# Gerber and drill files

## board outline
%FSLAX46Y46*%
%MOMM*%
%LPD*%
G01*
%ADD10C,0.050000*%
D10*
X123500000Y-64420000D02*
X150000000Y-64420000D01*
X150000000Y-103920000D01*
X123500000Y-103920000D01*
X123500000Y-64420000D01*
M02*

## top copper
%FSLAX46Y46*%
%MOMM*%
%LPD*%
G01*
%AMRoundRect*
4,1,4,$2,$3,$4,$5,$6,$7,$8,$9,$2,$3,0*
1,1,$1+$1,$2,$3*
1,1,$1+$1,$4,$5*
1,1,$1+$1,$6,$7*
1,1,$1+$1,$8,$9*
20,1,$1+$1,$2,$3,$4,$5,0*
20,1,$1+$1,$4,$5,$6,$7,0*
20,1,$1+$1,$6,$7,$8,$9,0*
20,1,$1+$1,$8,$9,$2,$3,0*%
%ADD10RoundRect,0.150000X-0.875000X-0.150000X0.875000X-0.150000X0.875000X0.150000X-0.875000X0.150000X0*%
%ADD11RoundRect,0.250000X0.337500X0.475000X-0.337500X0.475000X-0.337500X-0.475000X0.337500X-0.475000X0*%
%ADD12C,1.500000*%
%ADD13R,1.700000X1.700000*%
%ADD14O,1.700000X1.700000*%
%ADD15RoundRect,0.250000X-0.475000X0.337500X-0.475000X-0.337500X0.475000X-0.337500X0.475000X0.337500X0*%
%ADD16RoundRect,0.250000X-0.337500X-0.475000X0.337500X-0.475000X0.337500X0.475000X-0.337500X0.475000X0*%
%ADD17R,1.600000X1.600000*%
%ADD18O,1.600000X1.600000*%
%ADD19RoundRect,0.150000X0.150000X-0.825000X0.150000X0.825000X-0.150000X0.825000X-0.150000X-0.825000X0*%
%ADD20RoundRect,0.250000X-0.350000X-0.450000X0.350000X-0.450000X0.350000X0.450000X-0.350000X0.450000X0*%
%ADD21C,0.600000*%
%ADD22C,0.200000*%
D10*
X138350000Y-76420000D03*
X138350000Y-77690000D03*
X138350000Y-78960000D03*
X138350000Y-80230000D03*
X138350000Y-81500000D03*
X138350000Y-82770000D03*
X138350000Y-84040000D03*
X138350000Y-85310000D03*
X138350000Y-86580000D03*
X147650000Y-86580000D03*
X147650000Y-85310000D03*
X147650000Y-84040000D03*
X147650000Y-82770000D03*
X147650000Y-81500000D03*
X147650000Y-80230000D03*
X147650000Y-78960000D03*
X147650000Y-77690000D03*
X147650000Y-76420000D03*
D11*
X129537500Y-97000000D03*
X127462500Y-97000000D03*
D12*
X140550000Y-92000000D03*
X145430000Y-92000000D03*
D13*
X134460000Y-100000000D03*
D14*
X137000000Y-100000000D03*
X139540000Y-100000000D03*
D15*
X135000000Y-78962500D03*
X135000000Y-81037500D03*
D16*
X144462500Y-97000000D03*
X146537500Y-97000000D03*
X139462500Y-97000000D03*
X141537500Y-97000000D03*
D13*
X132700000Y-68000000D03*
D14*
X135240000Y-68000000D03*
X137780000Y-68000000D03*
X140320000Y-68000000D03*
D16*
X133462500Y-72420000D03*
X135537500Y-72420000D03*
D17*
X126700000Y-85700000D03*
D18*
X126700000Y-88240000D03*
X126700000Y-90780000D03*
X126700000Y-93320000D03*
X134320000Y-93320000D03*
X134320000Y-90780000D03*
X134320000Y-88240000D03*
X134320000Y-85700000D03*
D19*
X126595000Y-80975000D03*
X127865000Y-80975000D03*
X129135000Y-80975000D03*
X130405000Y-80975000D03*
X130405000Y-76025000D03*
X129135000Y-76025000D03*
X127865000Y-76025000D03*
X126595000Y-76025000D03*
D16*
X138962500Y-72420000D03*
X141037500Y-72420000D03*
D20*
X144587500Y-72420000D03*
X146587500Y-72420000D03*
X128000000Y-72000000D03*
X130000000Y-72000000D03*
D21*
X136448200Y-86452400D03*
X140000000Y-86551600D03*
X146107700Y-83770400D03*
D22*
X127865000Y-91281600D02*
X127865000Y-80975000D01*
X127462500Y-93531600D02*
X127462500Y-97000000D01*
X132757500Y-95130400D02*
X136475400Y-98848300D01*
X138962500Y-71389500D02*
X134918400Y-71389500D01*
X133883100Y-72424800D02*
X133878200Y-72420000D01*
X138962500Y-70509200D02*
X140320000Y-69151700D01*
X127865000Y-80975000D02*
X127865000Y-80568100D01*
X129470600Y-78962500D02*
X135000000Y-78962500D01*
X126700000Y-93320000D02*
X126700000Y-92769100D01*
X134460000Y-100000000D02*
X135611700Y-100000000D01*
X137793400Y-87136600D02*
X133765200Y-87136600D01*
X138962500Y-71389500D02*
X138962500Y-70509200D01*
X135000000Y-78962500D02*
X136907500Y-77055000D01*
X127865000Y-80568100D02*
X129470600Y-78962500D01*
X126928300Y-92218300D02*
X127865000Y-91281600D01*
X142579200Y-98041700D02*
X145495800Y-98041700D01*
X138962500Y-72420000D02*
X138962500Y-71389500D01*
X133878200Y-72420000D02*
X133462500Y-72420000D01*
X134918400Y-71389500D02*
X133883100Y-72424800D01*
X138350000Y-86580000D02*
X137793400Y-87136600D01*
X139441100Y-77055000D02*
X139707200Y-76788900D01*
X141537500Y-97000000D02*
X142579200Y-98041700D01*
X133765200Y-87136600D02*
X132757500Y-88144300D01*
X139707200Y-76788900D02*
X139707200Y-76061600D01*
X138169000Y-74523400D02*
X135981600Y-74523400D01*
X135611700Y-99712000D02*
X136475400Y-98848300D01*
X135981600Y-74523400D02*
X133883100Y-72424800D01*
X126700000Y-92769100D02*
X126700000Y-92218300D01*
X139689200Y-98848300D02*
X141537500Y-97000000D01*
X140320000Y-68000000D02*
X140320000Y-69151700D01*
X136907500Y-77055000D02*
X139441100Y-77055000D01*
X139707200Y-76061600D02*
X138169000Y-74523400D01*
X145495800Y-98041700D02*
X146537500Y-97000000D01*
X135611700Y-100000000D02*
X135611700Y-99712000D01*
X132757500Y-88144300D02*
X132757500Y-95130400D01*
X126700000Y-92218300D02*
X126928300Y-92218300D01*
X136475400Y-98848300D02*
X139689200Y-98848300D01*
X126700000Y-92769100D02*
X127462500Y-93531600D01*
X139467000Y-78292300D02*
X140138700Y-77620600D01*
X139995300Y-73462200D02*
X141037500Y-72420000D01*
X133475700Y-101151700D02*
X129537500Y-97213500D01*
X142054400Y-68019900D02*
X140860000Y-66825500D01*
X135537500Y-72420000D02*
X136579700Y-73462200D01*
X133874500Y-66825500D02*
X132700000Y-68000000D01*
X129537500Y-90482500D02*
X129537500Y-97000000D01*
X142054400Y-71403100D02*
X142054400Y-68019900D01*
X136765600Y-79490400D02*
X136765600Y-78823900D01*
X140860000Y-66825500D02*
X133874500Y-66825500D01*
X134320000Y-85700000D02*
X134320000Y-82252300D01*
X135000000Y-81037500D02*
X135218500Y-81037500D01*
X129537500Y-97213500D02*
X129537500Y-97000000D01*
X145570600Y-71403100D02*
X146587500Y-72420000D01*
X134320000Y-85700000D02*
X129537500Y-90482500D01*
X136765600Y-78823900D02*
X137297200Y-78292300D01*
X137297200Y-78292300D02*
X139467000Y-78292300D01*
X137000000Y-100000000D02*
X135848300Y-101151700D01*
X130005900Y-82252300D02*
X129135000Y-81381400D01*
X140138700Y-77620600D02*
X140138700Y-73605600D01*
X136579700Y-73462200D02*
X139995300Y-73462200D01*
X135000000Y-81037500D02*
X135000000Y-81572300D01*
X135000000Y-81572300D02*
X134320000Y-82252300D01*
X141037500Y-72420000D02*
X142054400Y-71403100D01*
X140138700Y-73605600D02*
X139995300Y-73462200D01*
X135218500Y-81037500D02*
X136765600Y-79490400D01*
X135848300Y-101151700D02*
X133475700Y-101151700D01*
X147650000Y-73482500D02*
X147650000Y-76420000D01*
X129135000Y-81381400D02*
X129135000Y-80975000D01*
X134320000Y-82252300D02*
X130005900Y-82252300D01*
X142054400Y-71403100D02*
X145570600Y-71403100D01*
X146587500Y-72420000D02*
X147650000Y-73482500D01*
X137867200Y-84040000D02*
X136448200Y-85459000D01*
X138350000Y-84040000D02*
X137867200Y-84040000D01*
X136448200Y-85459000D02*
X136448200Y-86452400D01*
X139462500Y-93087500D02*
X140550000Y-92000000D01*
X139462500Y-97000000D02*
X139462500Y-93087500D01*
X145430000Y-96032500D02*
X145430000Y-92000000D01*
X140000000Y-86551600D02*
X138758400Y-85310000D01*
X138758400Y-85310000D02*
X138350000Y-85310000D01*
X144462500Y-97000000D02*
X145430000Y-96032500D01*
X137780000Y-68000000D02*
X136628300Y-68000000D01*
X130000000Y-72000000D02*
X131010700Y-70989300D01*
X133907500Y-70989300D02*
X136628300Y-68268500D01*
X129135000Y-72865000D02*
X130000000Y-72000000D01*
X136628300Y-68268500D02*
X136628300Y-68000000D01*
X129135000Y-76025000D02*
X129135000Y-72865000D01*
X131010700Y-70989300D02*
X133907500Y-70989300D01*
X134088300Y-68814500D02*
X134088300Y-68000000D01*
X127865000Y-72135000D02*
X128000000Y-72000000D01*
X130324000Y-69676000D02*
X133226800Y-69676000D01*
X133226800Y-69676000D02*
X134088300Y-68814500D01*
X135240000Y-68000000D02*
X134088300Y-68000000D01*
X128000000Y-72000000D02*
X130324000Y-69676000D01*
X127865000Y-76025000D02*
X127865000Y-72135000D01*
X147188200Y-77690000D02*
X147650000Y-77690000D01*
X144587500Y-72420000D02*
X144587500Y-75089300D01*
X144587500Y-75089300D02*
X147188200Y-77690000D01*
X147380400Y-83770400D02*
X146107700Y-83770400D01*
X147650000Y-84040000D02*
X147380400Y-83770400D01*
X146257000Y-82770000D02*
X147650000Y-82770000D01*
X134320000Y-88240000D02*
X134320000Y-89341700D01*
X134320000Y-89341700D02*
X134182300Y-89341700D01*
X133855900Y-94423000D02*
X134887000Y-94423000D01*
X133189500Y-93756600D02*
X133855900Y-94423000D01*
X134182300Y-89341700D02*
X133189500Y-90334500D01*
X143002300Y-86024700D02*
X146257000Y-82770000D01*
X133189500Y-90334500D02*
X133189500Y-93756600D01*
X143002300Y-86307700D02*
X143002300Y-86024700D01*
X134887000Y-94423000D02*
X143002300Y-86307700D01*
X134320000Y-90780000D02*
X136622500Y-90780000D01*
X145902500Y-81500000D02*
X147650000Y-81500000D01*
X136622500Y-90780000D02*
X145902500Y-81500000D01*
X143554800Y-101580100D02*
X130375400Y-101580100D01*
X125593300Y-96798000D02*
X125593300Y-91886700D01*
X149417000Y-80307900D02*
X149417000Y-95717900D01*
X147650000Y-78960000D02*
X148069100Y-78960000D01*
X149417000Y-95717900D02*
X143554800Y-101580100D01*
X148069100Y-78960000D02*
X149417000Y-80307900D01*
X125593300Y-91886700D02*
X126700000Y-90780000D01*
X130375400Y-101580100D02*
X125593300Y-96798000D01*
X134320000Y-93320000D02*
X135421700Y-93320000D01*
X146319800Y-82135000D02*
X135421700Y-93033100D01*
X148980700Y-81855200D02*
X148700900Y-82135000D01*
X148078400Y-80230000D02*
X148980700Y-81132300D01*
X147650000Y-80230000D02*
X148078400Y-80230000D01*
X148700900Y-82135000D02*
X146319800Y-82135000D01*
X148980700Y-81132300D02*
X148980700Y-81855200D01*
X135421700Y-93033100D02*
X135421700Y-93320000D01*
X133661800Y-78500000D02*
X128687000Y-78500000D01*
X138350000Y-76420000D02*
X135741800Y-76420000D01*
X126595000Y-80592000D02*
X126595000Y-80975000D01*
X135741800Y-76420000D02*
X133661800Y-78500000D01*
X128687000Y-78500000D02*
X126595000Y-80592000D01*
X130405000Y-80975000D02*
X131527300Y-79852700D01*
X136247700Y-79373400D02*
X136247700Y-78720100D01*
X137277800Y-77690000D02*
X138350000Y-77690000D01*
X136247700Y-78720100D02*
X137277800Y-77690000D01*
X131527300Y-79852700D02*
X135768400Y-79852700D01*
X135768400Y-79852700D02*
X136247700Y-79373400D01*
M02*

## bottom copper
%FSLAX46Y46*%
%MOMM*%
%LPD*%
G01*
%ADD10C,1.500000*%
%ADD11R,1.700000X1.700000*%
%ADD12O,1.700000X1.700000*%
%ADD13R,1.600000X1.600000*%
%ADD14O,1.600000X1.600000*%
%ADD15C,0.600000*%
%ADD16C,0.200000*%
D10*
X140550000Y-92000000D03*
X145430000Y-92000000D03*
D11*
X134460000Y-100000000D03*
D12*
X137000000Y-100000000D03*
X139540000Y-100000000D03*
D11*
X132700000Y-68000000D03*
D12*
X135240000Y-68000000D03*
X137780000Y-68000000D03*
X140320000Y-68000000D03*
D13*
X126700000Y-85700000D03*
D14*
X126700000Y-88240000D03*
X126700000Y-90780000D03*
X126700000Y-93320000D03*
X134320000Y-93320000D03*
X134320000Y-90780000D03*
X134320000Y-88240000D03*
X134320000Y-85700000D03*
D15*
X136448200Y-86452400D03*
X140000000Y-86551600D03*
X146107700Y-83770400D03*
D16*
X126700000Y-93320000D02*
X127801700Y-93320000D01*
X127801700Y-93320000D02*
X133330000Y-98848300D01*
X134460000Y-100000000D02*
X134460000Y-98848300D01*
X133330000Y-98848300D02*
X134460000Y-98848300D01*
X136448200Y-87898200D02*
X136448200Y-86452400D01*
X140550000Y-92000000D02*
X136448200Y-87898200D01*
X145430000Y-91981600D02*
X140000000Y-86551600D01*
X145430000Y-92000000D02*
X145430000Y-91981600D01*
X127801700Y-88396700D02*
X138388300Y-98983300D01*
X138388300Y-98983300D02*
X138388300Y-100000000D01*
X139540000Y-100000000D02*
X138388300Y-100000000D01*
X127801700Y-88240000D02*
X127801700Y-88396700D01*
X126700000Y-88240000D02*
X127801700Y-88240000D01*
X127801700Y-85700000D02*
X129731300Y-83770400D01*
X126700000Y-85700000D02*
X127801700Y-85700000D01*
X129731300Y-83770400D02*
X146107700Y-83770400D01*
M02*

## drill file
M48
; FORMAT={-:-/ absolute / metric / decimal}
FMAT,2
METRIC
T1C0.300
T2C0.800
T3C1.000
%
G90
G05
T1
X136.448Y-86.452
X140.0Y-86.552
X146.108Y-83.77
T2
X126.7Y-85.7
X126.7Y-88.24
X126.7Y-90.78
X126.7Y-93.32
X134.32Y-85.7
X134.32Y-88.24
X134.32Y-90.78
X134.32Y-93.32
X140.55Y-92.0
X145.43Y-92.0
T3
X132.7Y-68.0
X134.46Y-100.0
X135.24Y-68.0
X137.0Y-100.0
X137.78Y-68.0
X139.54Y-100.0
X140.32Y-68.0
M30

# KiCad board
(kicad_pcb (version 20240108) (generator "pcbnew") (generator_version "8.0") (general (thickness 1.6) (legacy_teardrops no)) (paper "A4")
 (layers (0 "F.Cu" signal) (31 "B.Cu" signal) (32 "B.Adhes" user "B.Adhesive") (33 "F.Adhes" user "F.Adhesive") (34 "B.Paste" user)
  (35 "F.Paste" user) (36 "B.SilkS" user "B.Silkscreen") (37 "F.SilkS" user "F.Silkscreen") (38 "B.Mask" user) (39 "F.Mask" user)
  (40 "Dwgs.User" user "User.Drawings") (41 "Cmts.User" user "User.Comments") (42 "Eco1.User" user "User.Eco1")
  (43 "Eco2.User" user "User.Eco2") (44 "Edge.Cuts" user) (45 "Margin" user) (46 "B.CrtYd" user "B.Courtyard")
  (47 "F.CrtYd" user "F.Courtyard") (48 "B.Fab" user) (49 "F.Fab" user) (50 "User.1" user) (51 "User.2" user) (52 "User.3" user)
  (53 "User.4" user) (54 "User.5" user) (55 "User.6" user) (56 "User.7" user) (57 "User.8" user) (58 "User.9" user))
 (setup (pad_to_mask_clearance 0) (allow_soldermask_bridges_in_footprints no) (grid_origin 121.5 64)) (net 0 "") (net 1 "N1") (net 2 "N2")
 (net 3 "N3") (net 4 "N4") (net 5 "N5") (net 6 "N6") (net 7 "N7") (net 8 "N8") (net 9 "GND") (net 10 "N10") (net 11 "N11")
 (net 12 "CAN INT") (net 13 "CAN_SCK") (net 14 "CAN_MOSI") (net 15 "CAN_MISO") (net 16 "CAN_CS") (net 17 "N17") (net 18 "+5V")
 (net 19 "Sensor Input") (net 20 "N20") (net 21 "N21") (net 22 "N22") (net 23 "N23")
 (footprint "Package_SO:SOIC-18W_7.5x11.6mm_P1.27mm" (layer "F.Cu") (at 143 81.5)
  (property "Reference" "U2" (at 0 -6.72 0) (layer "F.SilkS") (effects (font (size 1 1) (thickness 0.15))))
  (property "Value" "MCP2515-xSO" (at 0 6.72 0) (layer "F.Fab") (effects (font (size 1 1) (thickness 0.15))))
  (pad "1" smd roundrect (at -4.65 -5.08) (size 2.05 0.6) (layers "F.Cu" "F.Paste" "F.Mask") (roundrect_rratio 0.25) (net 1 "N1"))
  (pad "2" smd roundrect (at -4.65 -3.81) (size 2.05 0.6) (layers "F.Cu" "F.Paste" "F.Mask") (roundrect_rratio 0.25) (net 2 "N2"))
  (pad "3" smd roundrect (at -4.65 -2.54) (size 2.05 0.6) (layers "F.Cu" "F.Paste" "F.Mask") (roundrect_rratio 0.25) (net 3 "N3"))
  (pad "4" smd roundrect (at -4.65 -1.27) (size 2.05 0.6) (layers "F.Cu" "F.Paste" "F.Mask") (roundrect_rratio 0.25) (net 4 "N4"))
  (pad "5" smd roundrect (at -4.65 0) (size 2.05 0.6) (layers "F.Cu" "F.Paste" "F.Mask") (roundrect_rratio 0.25) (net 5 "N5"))
  (pad "6" smd roundrect (at -4.65 1.27) (size 2.05 0.6) (layers "F.Cu" "F.Paste" "F.Mask") (roundrect_rratio 0.25) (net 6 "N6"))
  (pad "7" smd roundrect (at -4.65 2.54) (size 2.05 0.6) (layers "F.Cu" "F.Paste" "F.Mask") (roundrect_rratio 0.25) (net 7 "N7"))
  (pad "8" smd roundrect (at -4.65 3.81) (size 2.05 0.6) (layers "F.Cu" "F.Paste" "F.Mask") (roundrect_rratio 0.25) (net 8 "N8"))
  (pad "9" smd roundrect (at -4.65 5.08) (size 2.05 0.6) (layers "F.Cu" "F.Paste" "F.Mask") (roundrect_rratio 0.25) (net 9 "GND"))
  (pad "10" smd roundrect (at 4.65 5.08) (size 2.05 0.6) (layers "F.Cu" "F.Paste" "F.Mask") (roundrect_rratio 0.25) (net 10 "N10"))
  (pad "11" smd roundrect (at 4.65 3.81) (size 2.05 0.6) (layers "F.Cu" "F.Paste" "F.Mask") (roundrect_rratio 0.25) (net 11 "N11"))
  (pad "12" smd roundrect (at 4.65 2.54) (size 2.05 0.6) (layers "F.Cu" "F.Paste" "F.Mask") (roundrect_rratio 0.25) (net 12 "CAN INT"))
  (pad "13" smd roundrect (at 4.65 1.27) (size 2.05 0.6) (layers "F.Cu" "F.Paste" "F.Mask") (roundrect_rratio 0.25) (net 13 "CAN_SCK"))
  (pad "14" smd roundrect (at 4.65 0) (size 2.05 0.6) (layers "F.Cu" "F.Paste" "F.Mask") (roundrect_rratio 0.25) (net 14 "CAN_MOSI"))
  (pad "15" smd roundrect (at 4.65 -1.27) (size 2.05 0.6) (layers "F.Cu" "F.Paste" "F.Mask") (roundrect_rratio 0.25) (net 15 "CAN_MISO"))
  (pad "16" smd roundrect (at 4.65 -2.54) (size 2.05 0.6) (layers "F.Cu" "F.Paste" "F.Mask") (roundrect_rratio 0.25) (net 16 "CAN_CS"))
  (pad "17" smd roundrect (at 4.65 -3.81) (size 2.05 0.6) (layers "F.Cu" "F.Paste" "F.Mask") (roundrect_rratio 0.25) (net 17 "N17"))
  (pad "18" smd roundrect (at 4.65 -5.08) (size 2.05 0.6) (layers "F.Cu" "F.Paste" "F.Mask") (roundrect_rratio 0.25) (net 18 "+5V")))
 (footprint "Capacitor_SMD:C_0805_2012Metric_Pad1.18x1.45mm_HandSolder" (layer "F.Cu") (at 128.5 97 180)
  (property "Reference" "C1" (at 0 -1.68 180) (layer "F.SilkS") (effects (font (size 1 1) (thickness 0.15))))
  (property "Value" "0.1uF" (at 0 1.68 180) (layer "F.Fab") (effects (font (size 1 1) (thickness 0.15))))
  (pad "1" smd roundrect (at -1.0375 0 180) (size 1.175 1.45) (layers "F.Cu" "F.Paste" "F.Mask") (roundrect_rratio 0.212766) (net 18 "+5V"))
  (pad "2" smd roundrect (at 1.0375 0 180) (size 1.175 1.45) (layers "F.Cu" "F.Paste" "F.Mask") (roundrect_rratio 0.212766) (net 9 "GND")))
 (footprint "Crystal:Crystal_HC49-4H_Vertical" (layer "F.Cu") (at 140.55 92)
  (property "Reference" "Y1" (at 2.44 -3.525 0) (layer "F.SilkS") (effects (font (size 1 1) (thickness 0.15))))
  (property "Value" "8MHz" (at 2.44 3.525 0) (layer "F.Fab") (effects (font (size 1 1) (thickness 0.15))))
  (pad "1" thru_hole circle (at 0 0) (size 1.5 1.5) (drill 0.8) (layers "*.Cu" "*.Mask") (remove_unused_layers no) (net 7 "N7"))
  (pad "2" thru_hole circle (at 4.88 0) (size 1.5 1.5) (drill 0.8) (layers "*.Cu" "*.Mask") (remove_unused_layers no) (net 8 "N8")))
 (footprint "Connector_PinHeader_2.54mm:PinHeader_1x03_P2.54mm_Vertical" (layer "F.Cu") (at 134.46 100 90)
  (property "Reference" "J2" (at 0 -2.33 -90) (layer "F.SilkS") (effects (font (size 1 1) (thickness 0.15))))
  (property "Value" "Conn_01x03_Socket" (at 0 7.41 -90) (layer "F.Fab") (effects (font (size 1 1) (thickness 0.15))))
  (pad "1" thru_hole rect (at 0 0 90) (size 1.7 1.7) (drill 1) (layers "*.Cu" "*.Mask") (remove_unused_layers no) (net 9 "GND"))
  (pad "2" thru_hole oval (at 0 2.54 90) (size 1.7 1.7) (drill 1) (layers "*.Cu" "*.Mask") (remove_unused_layers no) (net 18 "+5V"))
  (pad "3" thru_hole oval (at 0 5.08 90) (size 1.7 1.7) (drill 1) (layers "*.Cu" "*.Mask") (remove_unused_layers no) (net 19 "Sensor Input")))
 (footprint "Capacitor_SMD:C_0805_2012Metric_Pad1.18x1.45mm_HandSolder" (layer "F.Cu") (at 135 80 -90)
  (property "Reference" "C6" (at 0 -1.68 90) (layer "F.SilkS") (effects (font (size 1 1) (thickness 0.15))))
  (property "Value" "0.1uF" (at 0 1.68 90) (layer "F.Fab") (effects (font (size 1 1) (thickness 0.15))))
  (pad "1" smd roundrect (at -1.0375 0 270) (size 1.175 1.45) (layers "F.Cu" "F.Paste" "F.Mask") (roundrect_rratio 0.212766) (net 9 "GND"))
  (pad "2" smd roundrect (at 1.0375 0 270) (size 1.175 1.45) (layers "F.Cu" "F.Paste" "F.Mask") (roundrect_rratio 0.212766) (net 18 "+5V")))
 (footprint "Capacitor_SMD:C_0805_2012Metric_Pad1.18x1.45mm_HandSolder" (layer "F.Cu") (at 145.5 97)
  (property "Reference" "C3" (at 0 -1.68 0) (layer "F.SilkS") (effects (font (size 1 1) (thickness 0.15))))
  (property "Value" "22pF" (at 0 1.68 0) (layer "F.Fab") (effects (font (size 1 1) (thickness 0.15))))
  (pad "1" smd roundrect (at -1.0375 0) (size 1.175 1.45) (layers "F.Cu" "F.Paste" "F.Mask") (roundrect_rratio 0.212766) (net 8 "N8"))
  (pad "2" smd roundrect (at 1.0375 0) (size 1.175 1.45) (layers "F.Cu" "F.Paste" "F.Mask") (roundrect_rratio 0.212766) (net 9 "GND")))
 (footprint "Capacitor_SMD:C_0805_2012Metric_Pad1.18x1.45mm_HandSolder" (layer "F.Cu") (at 140.5 97)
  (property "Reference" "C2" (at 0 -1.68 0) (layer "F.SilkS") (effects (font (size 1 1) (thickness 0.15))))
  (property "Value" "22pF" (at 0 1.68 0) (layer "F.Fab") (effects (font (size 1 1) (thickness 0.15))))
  (pad "1" smd roundrect (at -1.0375 0) (size 1.175 1.45) (layers "F.Cu" "F.Paste" "F.Mask") (roundrect_rratio 0.212766) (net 7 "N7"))
  (pad "2" smd roundrect (at 1.0375 0) (size 1.175 1.45) (layers "F.Cu" "F.Paste" "F.Mask") (roundrect_rratio 0.212766) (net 9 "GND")))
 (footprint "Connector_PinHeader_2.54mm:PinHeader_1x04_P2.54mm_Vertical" (layer "F.Cu") (at 132.7 68 90)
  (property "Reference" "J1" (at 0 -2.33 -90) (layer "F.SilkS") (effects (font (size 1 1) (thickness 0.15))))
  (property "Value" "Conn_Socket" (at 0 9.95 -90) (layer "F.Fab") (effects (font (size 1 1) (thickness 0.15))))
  (pad "1" thru_hole rect (at 0 0 90) (size 1.7 1.7) (drill 1) (layers "*.Cu" "*.Mask") (remove_unused_layers no) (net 18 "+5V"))
  (pad "2" thru_hole oval (at 0 2.54 90) (size 1.7 1.7) (drill 1) (layers "*.Cu" "*.Mask") (remove_unused_layers no) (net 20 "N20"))
  (pad "3" thru_hole oval (at 0 5.08 90) (size 1.7 1.7) (drill 1) (layers "*.Cu" "*.Mask") (remove_unused_layers no) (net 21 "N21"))
  (pad "4" thru_hole oval (at 0 7.62 90) (size 1.7 1.7) (drill 1) (layers "*.Cu" "*.Mask") (remove_unused_layers no) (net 9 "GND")))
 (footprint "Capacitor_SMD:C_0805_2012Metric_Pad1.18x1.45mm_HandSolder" (layer "F.Cu") (at 134.5 72.42)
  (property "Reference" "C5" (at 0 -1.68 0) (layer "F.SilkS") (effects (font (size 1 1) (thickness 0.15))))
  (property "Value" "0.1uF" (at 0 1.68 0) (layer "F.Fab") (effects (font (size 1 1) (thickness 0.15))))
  (pad "1" smd roundrect (at -1.0375 0) (size 1.175 1.45) (layers "F.Cu" "F.Paste" "F.Mask") (roundrect_rratio 0.212766) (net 9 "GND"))
  (pad "2" smd roundrect (at 1.0375 0) (size 1.175 1.45) (layers "F.Cu" "F.Paste" "F.Mask") (roundrect_rratio 0.212766) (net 18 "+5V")))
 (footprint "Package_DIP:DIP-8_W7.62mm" (layer "F.Cu") (at 126.7 85.7)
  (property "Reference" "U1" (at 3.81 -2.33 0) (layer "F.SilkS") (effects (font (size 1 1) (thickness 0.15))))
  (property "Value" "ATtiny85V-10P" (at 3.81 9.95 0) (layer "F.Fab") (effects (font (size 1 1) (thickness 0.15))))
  (pad "1" thru_hole rect (at 0 0) (size 1.6 1.6) (drill 0.8) (layers "*.Cu" "*.Mask") (remove_unused_layers no) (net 12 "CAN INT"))
  (pad "2" thru_hole oval (at 0 2.54) (size 1.6 1.6) (drill 0.8) (layers "*.Cu" "*.Mask") (remove_unused_layers no) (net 19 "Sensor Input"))
  (pad "3" thru_hole oval (at 0 5.08) (size 1.6 1.6) (drill 0.8) (layers "*.Cu" "*.Mask") (remove_unused_layers no) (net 16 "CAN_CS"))
  (pad "4" thru_hole oval (at 0 7.62) (size 1.6 1.6) (drill 0.8) (layers "*.Cu" "*.Mask") (remove_unused_layers no) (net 9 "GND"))
  (pad "5" thru_hole oval (at 7.62 7.62) (size 1.6 1.6) (drill 0.8) (layers "*.Cu" "*.Mask") (remove_unused_layers no) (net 15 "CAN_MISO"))
  (pad "6" thru_hole oval (at 7.62 5.08) (size 1.6 1.6) (drill 0.8) (layers "*.Cu" "*.Mask") (remove_unused_layers no) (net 14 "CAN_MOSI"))
  (pad "7" thru_hole oval (at 7.62 2.54) (size 1.6 1.6) (drill 0.8) (layers "*.Cu" "*.Mask") (remove_unused_layers no) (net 13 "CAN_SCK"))
  (pad "8" thru_hole oval (at 7.62 0) (size 1.6 1.6) (drill 0.8) (layers "*.Cu" "*.Mask") (remove_unused_layers no) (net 18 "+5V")))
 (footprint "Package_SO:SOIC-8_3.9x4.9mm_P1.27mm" (layer "F.Cu") (at 128.5 78.5 90)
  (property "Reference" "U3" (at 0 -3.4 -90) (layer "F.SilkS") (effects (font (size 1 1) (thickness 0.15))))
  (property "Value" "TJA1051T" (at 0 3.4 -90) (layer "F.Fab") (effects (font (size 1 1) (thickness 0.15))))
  (pad "1" smd roundrect (at -2.475 -1.905 90) (size 1.95 0.6) (layers "F.Cu" "F.Paste" "F.Mask") (roundrect_rratio 0.25) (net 1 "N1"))
  (pad "2" smd roundrect (at -2.475 -0.635 90) (size 1.95 0.6) (layers "F.Cu" "F.Paste" "F.Mask") (roundrect_rratio 0.25) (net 9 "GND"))
  (pad "3" smd roundrect (at -2.475 0.635 90) (size 1.95 0.6) (layers "F.Cu" "F.Paste" "F.Mask") (roundrect_rratio 0.25) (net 18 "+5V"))
  (pad "4" smd roundrect (at -2.475 1.905 90) (size 1.95 0.6) (layers "F.Cu" "F.Paste" "F.Mask") (roundrect_rratio 0.25) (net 2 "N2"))
  (pad "5" smd roundrect (at 2.475 1.905 90) (size 1.95 0.6) (layers "F.Cu" "F.Paste" "F.Mask") (roundrect_rratio 0.25) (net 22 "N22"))
  (pad "6" smd roundrect (at 2.475 0.635 90) (size 1.95 0.6) (layers "F.Cu" "F.Paste" "F.Mask") (roundrect_rratio 0.25) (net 21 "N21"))
  (pad "7" smd roundrect (at 2.475 -0.635 90) (size 1.95 0.6) (layers "F.Cu" "F.Paste" "F.Mask") (roundrect_rratio 0.25) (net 20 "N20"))
  (pad "8" smd roundrect (at 2.475 -1.905 90) (size 1.95 0.6) (layers "F.Cu" "F.Paste" "F.Mask") (roundrect_rratio 0.25) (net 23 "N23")))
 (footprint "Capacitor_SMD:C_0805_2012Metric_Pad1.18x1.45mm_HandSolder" (layer "F.Cu") (at 140 72.42)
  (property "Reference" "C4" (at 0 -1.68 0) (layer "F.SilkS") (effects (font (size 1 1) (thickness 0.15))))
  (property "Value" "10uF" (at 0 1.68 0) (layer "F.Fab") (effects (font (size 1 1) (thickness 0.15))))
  (pad "1" smd roundrect (at -1.0375 0) (size 1.175 1.45) (layers "F.Cu" "F.Paste" "F.Mask") (roundrect_rratio 0.212766) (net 9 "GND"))
  (pad "2" smd roundrect (at 1.0375 0) (size 1.175 1.45) (layers "F.Cu" "F.Paste" "F.Mask") (roundrect_rratio 0.212766) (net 18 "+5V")))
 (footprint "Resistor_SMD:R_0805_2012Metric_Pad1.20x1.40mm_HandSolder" (layer "F.Cu") (at 145.5875 72.42)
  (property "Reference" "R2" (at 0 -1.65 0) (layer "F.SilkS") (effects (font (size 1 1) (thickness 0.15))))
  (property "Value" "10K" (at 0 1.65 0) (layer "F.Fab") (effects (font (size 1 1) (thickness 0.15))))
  (pad "1" smd roundrect (at -1 0) (size 1.2 1.4) (layers "F.Cu" "F.Paste" "F.Mask") (roundrect_rratio 0.208333) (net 17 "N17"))
  (pad "2" smd roundrect (at 1 0) (size 1.2 1.4) (layers "F.Cu" "F.Paste" "F.Mask") (roundrect_rratio 0.208333) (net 18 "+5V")))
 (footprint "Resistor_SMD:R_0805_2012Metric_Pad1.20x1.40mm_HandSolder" (layer "F.Cu") (at 129 72)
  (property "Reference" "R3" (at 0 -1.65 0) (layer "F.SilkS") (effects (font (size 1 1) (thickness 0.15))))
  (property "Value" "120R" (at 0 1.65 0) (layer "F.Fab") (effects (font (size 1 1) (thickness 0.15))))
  (pad "1" smd roundrect (at -1 0) (size 1.2 1.4) (layers "F.Cu" "F.Paste" "F.Mask") (roundrect_rratio 0.208333) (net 20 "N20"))
  (pad "2" smd roundrect (at 1 0) (size 1.2 1.4) (layers "F.Cu" "F.Paste" "F.Mask") (roundrect_rratio 0.208333) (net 21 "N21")))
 (gr_rect (start 123.5 64.42) (end 150 103.92) (stroke (width 0.05) (type default)) (fill none) (layer "Edge.Cuts"))
 (segment (start 127.865 91.2816) (end 127.865 80.975) (width 0.2) (layer "F.Cu") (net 9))
 (segment (start 127.4625 93.5316) (end 127.4625 97) (width 0.2) (layer "F.Cu") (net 9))
 (segment (start 132.7575 95.1304) (end 136.4754 98.8483) (width 0.2) (layer "F.Cu") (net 9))
 (segment (start 138.9625 71.3895) (end 134.9184 71.3895) (width 0.2) (layer "F.Cu") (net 9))
 (segment (start 133.8831 72.4248) (end 133.8782 72.42) (width 0.2) (layer "F.Cu") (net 9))
 (segment (start 138.9625 70.5092) (end 140.32 69.1517) (width 0.2) (layer "F.Cu") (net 9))
 (segment (start 127.865 80.975) (end 127.865 80.5681) (width 0.2) (layer "F.Cu") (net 9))
 (segment (start 129.4706 78.9625) (end 135 78.9625) (width 0.2) (layer "F.Cu") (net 9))
 (segment (start 126.7 93.32) (end 126.7 92.7691) (width 0.2) (layer "F.Cu") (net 9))
 (segment (start 134.46 100) (end 135.6117 100) (width 0.2) (layer "F.Cu") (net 9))
 (segment (start 137.7934 87.1366) (end 133.7652 87.1366) (width 0.2) (layer "F.Cu") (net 9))
 (segment (start 138.9625 71.3895) (end 138.9625 70.5092) (width 0.2) (layer "F.Cu") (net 9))
 (segment (start 135 78.9625) (end 136.9075 77.055) (width 0.2) (layer "F.Cu") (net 9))
 (segment (start 127.865 80.5681) (end 129.4706 78.9625) (width 0.2) (layer "F.Cu") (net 9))
 (segment (start 126.9283 92.2183) (end 127.865 91.2816) (width 0.2) (layer "F.Cu") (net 9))
 (segment (start 142.5792 98.0417) (end 145.4958 98.0417) (width 0.2) (layer "F.Cu") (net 9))
 (segment (start 138.9625 72.42) (end 138.9625 71.3895) (width 0.2) (layer "F.Cu") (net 9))
 (segment (start 133.8782 72.42) (end 133.4625 72.42) (width 0.2) (layer "F.Cu") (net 9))
 (segment (start 134.9184 71.3895) (end 133.8831 72.4248) (width 0.2) (layer "F.Cu") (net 9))
 (segment (start 138.35 86.58) (end 137.7934 87.1366) (width 0.2) (layer "F.Cu") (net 9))
 (segment (start 139.4411 77.055) (end 139.7072 76.7889) (width 0.2) (layer "F.Cu") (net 9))
 (segment (start 141.5375 97) (end 142.5792 98.0417) (width 0.2) (layer "F.Cu") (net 9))
 (segment (start 133.7652 87.1366) (end 132.7575 88.1443) (width 0.2) (layer "F.Cu") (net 9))
 (segment (start 139.7072 76.7889) (end 139.7072 76.0616) (width 0.2) (layer "F.Cu") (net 9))
 (segment (start 138.169 74.5234) (end 135.9816 74.5234) (width 0.2) (layer "F.Cu") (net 9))
 (segment (start 135.6117 99.712) (end 136.4754 98.8483) (width 0.2) (layer "F.Cu") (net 9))
 (segment (start 135.9816 74.5234) (end 133.8831 72.4248) (width 0.2) (layer "F.Cu") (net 9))
 (segment (start 126.7 92.7691) (end 126.7 92.2183) (width 0.2) (layer "F.Cu") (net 9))
 (segment (start 139.6892 98.8483) (end 141.5375 97) (width 0.2) (layer "F.Cu") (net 9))
 (segment (start 140.32 68) (end 140.32 69.1517) (width 0.2) (layer "F.Cu") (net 9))
 (segment (start 136.9075 77.055) (end 139.4411 77.055) (width 0.2) (layer "F.Cu") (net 9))
 (segment (start 139.7072 76.0616) (end 138.169 74.5234) (width 0.2) (layer "F.Cu") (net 9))
 (segment (start 145.4958 98.0417) (end 146.5375 97) (width 0.2) (layer "F.Cu") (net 9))
 (segment (start 135.6117 100) (end 135.6117 99.712) (width 0.2) (layer "F.Cu") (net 9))
 (segment (start 132.7575 88.1443) (end 132.7575 95.1304) (width 0.2) (layer "F.Cu") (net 9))
 (segment (start 126.7 92.2183) (end 126.9283 92.2183) (width 0.2) (layer "F.Cu") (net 9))
 (segment (start 136.4754 98.8483) (end 139.6892 98.8483) (width 0.2) (layer "F.Cu") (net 9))
 (segment (start 126.7 92.7691) (end 127.4625 93.5316) (width 0.2) (layer "F.Cu") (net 9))
 (segment (start 126.7 93.32) (end 127.8017 93.32) (width 0.2) (layer "B.Cu") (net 9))
 (segment (start 127.8017 93.32) (end 133.33 98.8483) (width 0.2) (layer "B.Cu") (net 9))
 (segment (start 134.46 100) (end 134.46 98.8483) (width 0.2) (layer "B.Cu") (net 9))
 (segment (start 133.33 98.8483) (end 134.46 98.8483) (width 0.2) (layer "B.Cu") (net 9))
 (segment (start 139.467 78.2923) (end 140.1387 77.6206) (width 0.2) (layer "F.Cu") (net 18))
 (segment (start 139.9953 73.4622) (end 141.0375 72.42) (width 0.2) (layer "F.Cu") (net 18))
 (segment (start 133.4757 101.1517) (end 129.5375 97.2135) (width 0.2) (layer "F.Cu") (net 18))
 (segment (start 142.0544 68.0199) (end 140.86 66.8255) (width 0.2) (layer "F.Cu") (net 18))
 (segment (start 135.5375 72.42) (end 136.5797 73.4622) (width 0.2) (layer "F.Cu") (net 18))
 (segment (start 133.8745 66.8255) (end 132.7 68) (width 0.2) (layer "F.Cu") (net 18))
 (segment (start 129.5375 90.4825) (end 129.5375 97) (width 0.2) (layer "F.Cu") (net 18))
 (segment (start 142.0544 71.4031) (end 142.0544 68.0199) (width 0.2) (layer "F.Cu") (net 18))
 (segment (start 136.7656 79.4904) (end 136.7656 78.8239) (width 0.2) (layer "F.Cu") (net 18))
 (segment (start 140.86 66.8255) (end 133.8745 66.8255) (width 0.2) (layer "F.Cu") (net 18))
 (segment (start 134.32 85.7) (end 134.32 82.2523) (width 0.2) (layer "F.Cu") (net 18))
 (segment (start 135 81.0375) (end 135.2185 81.0375) (width 0.2) (layer "F.Cu") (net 18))
 (segment (start 129.5375 97.2135) (end 129.5375 97) (width 0.2) (layer "F.Cu") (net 18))
 (segment (start 145.5706 71.4031) (end 146.5875 72.42) (width 0.2) (layer "F.Cu") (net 18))
 (segment (start 134.32 85.7) (end 129.5375 90.4825) (width 0.2) (layer "F.Cu") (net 18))
 (segment (start 136.7656 78.8239) (end 137.2972 78.2923) (width 0.2) (layer "F.Cu") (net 18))
 (segment (start 137.2972 78.2923) (end 139.467 78.2923) (width 0.2) (layer "F.Cu") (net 18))
 (segment (start 137 100) (end 135.8483 101.1517) (width 0.2) (layer "F.Cu") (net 18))
 (segment (start 130.0059 82.2523) (end 129.135 81.3814) (width 0.2) (layer "F.Cu") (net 18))
 (segment (start 140.1387 77.6206) (end 140.1387 73.6056) (width 0.2) (layer "F.Cu") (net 18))
 (segment (start 136.5797 73.4622) (end 139.9953 73.4622) (width 0.2) (layer "F.Cu") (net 18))
 (segment (start 135 81.0375) (end 135 81.5723) (width 0.2) (layer "F.Cu") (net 18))
 (segment (start 135 81.5723) (end 134.32 82.2523) (width 0.2) (layer "F.Cu") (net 18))
 (segment (start 141.0375 72.42) (end 142.0544 71.4031) (width 0.2) (layer "F.Cu") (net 18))
 (segment (start 140.1387 73.6056) (end 139.9953 73.4622) (width 0.2) (layer "F.Cu") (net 18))
 (segment (start 135.2185 81.0375) (end 136.7656 79.4904) (width 0.2) (layer "F.Cu") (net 18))
 (segment (start 135.8483 101.1517) (end 133.4757 101.1517) (width 0.2) (layer "F.Cu") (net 18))
 (segment (start 147.65 73.4825) (end 147.65 76.42) (width 0.2) (layer "F.Cu") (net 18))
 (segment (start 129.135 81.3814) (end 129.135 80.975) (width 0.2) (layer "F.Cu") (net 18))
 (segment (start 134.32 82.2523) (end 130.0059 82.2523) (width 0.2) (layer "F.Cu") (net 18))
 (segment (start 142.0544 71.4031) (end 145.5706 71.4031) (width 0.2) (layer "F.Cu") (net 18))
 (segment (start 146.5875 72.42) (end 147.65 73.4825) (width 0.2) (layer "F.Cu") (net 18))
 (segment (start 137.8672 84.04) (end 136.4482 85.459) (width 0.2) (layer "F.Cu") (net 7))
 (segment (start 138.35 84.04) (end 137.8672 84.04) (width 0.2) (layer "F.Cu") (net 7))
 (segment (start 136.4482 85.459) (end 136.4482 86.4524) (width 0.2) (layer "F.Cu") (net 7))
 (segment (start 139.4625 93.0875) (end 140.55 92) (width 0.2) (layer "F.Cu") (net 7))
 (segment (start 139.4625 97) (end 139.4625 93.0875) (width 0.2) (layer "F.Cu") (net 7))
 (via (at 136.4482 86.4524) (size 0.6) (drill 0.3) (layers "F.Cu" "B.Cu") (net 7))
 (segment (start 136.4482 87.8982) (end 136.4482 86.4524) (width 0.2) (layer "B.Cu") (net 7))
 (segment (start 140.55 92) (end 136.4482 87.8982) (width 0.2) (layer "B.Cu") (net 7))
 (segment (start 145.43 96.0325) (end 145.43 92) (width 0.2) (layer "F.Cu") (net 8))
 (segment (start 140 86.5516) (end 138.7584 85.31) (width 0.2) (layer "F.Cu") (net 8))
 (segment (start 138.7584 85.31) (end 138.35 85.31) (width 0.2) (layer "F.Cu") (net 8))
 (segment (start 144.4625 97) (end 145.43 96.0325) (width 0.2) (layer "F.Cu") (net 8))
 (via (at 140 86.5516) (size 0.6) (drill 0.3) (layers "F.Cu" "B.Cu") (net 8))
 (segment (start 145.43 91.9816) (end 140 86.5516) (width 0.2) (layer "B.Cu") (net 8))
 (segment (start 145.43 92) (end 145.43 91.9816) (width 0.2) (layer "B.Cu") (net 8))
 (segment (start 137.78 68) (end 136.6283 68) (width 0.2) (layer "F.Cu") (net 21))
 (segment (start 130 72) (end 131.0107 70.9893) (width 0.2) (layer "F.Cu") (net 21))
 (segment (start 133.9075 70.9893) (end 136.6283 68.2685) (width 0.2) (layer "F.Cu") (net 21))
 (segment (start 129.135 72.865) (end 130 72) (width 0.2) (layer "F.Cu") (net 21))
 (segment (start 136.6283 68.2685) (end 136.6283 68) (width 0.2) (layer "F.Cu") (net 21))
 (segment (start 129.135 76.025) (end 129.135 72.865) (width 0.2) (layer "F.Cu") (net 21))
 (segment (start 131.0107 70.9893) (end 133.9075 70.9893) (width 0.2) (layer "F.Cu") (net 21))
 (segment (start 134.0883 68.8145) (end 134.0883 68) (width 0.2) (layer "F.Cu") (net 20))
 (segment (start 127.865 72.135) (end 128 72) (width 0.2) (layer "F.Cu") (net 20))
 (segment (start 130.324 69.676) (end 133.2268 69.676) (width 0.2) (layer "F.Cu") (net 20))
 (segment (start 133.2268 69.676) (end 134.0883 68.8145) (width 0.2) (layer "F.Cu") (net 20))
 (segment (start 135.24 68) (end 134.0883 68) (width 0.2) (layer "F.Cu") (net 20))
 (segment (start 128 72) (end 130.324 69.676) (width 0.2) (layer "F.Cu") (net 20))
 (segment (start 127.865 76.025) (end 127.865 72.135) (width 0.2) (layer "F.Cu") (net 20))
 (segment (start 127.8017 88.3967) (end 138.3883 98.9833) (width 0.2) (layer "B.Cu") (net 19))
 (segment (start 138.3883 98.9833) (end 138.3883 100) (width 0.2) (layer "B.Cu") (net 19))
 (segment (start 139.54 100) (end 138.3883 100) (width 0.2) (layer "B.Cu") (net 19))
 (segment (start 127.8017 88.24) (end 127.8017 88.3967) (width 0.2) (layer "B.Cu") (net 19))
 (segment (start 126.7 88.24) (end 127.8017 88.24) (width 0.2) (layer "B.Cu") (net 19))
 (segment (start 147.1882 77.69) (end 147.65 77.69) (width 0.2) (layer "F.Cu") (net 17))
 (segment (start 144.5875 72.42) (end 144.5875 75.0893) (width 0.2) (layer "F.Cu") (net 17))
 (segment (start 144.5875 75.0893) (end 147.1882 77.69) (width 0.2) (layer "F.Cu") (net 17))
 (segment (start 147.3804 83.7704) (end 146.1077 83.7704) (width 0.2) (layer "F.Cu") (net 12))
 (segment (start 147.65 84.04) (end 147.3804 83.7704) (width 0.2) (layer "F.Cu") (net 12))
 (via (at 146.1077 83.7704) (size 0.6) (drill 0.3) (layers "F.Cu" "B.Cu") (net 12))
 (segment (start 127.8017 85.7) (end 129.7313 83.7704) (width 0.2) (layer "B.Cu") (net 12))
 (segment (start 126.7 85.7) (end 127.8017 85.7) (width 0.2) (layer "B.Cu") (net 12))
 (segment (start 129.7313 83.7704) (end 146.1077 83.7704) (width 0.2) (layer "B.Cu") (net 12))
 (segment (start 146.257 82.77) (end 147.65 82.77) (width 0.2) (layer "F.Cu") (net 13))
 (segment (start 134.32 88.24) (end 134.32 89.3417) (width 0.2) (layer "F.Cu") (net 13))
 (segment (start 134.32 89.3417) (end 134.1823 89.3417) (width 0.2) (layer "F.Cu") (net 13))
 (segment (start 133.8559 94.423) (end 134.887 94.423) (width 0.2) (layer "F.Cu") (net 13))
 (segment (start 133.1895 93.7566) (end 133.8559 94.423) (width 0.2) (layer "F.Cu") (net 13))
 (segment (start 134.1823 89.3417) (end 133.1895 90.3345) (width 0.2) (layer "F.Cu") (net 13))
 (segment (start 143.0023 86.0247) (end 146.257 82.77) (width 0.2) (layer "F.Cu") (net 13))
 (segment (start 133.1895 90.3345) (end 133.1895 93.7566) (width 0.2) (layer "F.Cu") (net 13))
 (segment (start 143.0023 86.3077) (end 143.0023 86.0247) (width 0.2) (layer "F.Cu") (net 13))
 (segment (start 134.887 94.423) (end 143.0023 86.3077) (width 0.2) (layer "F.Cu") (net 13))
 (segment (start 134.32 90.78) (end 136.6225 90.78) (width 0.2) (layer "F.Cu") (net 14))
 (segment (start 145.9025 81.5) (end 147.65 81.5) (width 0.2) (layer "F.Cu") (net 14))
 (segment (start 136.6225 90.78) (end 145.9025 81.5) (width 0.2) (layer "F.Cu") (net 14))
 (segment (start 143.5548 101.5801) (end 130.3754 101.5801) (width 0.2) (layer "F.Cu") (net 16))
 (segment (start 125.5933 96.798) (end 125.5933 91.8867) (width 0.2) (layer "F.Cu") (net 16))
 (segment (start 149.417 80.3079) (end 149.417 95.7179) (width 0.2) (layer "F.Cu") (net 16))
 (segment (start 147.65 78.96) (end 148.0691 78.96) (width 0.2) (layer "F.Cu") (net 16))
 (segment (start 149.417 95.7179) (end 143.5548 101.5801) (width 0.2) (layer "F.Cu") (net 16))
 (segment (start 148.0691 78.96) (end 149.417 80.3079) (width 0.2) (layer "F.Cu") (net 16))
 (segment (start 125.5933 91.8867) (end 126.7 90.78) (width 0.2) (layer "F.Cu") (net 16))
 (segment (start 130.3754 101.5801) (end 125.5933 96.798) (width 0.2) (layer "F.Cu") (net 16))
 (segment (start 134.32 93.32) (end 135.4217 93.32) (width 0.2) (layer "F.Cu") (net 15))
 (segment (start 146.3198 82.135) (end 135.4217 93.0331) (width 0.2) (layer "F.Cu") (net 15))
 (segment (start 148.9807 81.8552) (end 148.7009 82.135) (width 0.2) (layer "F.Cu") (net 15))
 (segment (start 148.0784 80.23) (end 148.9807 81.1323) (width 0.2) (layer "F.Cu") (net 15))
 (segment (start 147.65 80.23) (end 148.0784 80.23) (width 0.2) (layer "F.Cu") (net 15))
 (segment (start 148.7009 82.135) (end 146.3198 82.135) (width 0.2) (layer "F.Cu") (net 15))
 (segment (start 148.9807 81.1323) (end 148.9807 81.8552) (width 0.2) (layer "F.Cu") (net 15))
 (segment (start 135.4217 93.0331) (end 135.4217 93.32) (width 0.2) (layer "F.Cu") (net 15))
 (segment (start 133.6618 78.5) (end 128.687 78.5) (width 0.2) (layer "F.Cu") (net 1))
 (segment (start 138.35 76.42) (end 135.7418 76.42) (width 0.2) (layer "F.Cu") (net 1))
 (segment (start 126.595 80.592) (end 126.595 80.975) (width 0.2) (layer "F.Cu") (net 1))
 (segment (start 135.7418 76.42) (end 133.6618 78.5) (width 0.2) (layer "F.Cu") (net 1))
 (segment (start 128.687 78.5) (end 126.595 80.592) (width 0.2) (layer "F.Cu") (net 1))
 (segment (start 130.405 80.975) (end 131.5273 79.8527) (width 0.2) (layer "F.Cu") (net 2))
 (segment (start 136.2477 79.3734) (end 136.2477 78.7201) (width 0.2) (layer "F.Cu") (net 2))
 (segment (start 137.2778 77.69) (end 138.35 77.69) (width 0.2) (layer "F.Cu") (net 2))
 (segment (start 136.2477 78.7201) (end 137.2778 77.69) (width 0.2) (layer "F.Cu") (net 2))
 (segment (start 131.5273 79.8527) (end 135.7684 79.8527) (width 0.2) (layer "F.Cu") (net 2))
 (segment (start 135.7684 79.8527) (end 136.2477 79.3734) (width 0.2) (layer "F.Cu") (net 2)))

